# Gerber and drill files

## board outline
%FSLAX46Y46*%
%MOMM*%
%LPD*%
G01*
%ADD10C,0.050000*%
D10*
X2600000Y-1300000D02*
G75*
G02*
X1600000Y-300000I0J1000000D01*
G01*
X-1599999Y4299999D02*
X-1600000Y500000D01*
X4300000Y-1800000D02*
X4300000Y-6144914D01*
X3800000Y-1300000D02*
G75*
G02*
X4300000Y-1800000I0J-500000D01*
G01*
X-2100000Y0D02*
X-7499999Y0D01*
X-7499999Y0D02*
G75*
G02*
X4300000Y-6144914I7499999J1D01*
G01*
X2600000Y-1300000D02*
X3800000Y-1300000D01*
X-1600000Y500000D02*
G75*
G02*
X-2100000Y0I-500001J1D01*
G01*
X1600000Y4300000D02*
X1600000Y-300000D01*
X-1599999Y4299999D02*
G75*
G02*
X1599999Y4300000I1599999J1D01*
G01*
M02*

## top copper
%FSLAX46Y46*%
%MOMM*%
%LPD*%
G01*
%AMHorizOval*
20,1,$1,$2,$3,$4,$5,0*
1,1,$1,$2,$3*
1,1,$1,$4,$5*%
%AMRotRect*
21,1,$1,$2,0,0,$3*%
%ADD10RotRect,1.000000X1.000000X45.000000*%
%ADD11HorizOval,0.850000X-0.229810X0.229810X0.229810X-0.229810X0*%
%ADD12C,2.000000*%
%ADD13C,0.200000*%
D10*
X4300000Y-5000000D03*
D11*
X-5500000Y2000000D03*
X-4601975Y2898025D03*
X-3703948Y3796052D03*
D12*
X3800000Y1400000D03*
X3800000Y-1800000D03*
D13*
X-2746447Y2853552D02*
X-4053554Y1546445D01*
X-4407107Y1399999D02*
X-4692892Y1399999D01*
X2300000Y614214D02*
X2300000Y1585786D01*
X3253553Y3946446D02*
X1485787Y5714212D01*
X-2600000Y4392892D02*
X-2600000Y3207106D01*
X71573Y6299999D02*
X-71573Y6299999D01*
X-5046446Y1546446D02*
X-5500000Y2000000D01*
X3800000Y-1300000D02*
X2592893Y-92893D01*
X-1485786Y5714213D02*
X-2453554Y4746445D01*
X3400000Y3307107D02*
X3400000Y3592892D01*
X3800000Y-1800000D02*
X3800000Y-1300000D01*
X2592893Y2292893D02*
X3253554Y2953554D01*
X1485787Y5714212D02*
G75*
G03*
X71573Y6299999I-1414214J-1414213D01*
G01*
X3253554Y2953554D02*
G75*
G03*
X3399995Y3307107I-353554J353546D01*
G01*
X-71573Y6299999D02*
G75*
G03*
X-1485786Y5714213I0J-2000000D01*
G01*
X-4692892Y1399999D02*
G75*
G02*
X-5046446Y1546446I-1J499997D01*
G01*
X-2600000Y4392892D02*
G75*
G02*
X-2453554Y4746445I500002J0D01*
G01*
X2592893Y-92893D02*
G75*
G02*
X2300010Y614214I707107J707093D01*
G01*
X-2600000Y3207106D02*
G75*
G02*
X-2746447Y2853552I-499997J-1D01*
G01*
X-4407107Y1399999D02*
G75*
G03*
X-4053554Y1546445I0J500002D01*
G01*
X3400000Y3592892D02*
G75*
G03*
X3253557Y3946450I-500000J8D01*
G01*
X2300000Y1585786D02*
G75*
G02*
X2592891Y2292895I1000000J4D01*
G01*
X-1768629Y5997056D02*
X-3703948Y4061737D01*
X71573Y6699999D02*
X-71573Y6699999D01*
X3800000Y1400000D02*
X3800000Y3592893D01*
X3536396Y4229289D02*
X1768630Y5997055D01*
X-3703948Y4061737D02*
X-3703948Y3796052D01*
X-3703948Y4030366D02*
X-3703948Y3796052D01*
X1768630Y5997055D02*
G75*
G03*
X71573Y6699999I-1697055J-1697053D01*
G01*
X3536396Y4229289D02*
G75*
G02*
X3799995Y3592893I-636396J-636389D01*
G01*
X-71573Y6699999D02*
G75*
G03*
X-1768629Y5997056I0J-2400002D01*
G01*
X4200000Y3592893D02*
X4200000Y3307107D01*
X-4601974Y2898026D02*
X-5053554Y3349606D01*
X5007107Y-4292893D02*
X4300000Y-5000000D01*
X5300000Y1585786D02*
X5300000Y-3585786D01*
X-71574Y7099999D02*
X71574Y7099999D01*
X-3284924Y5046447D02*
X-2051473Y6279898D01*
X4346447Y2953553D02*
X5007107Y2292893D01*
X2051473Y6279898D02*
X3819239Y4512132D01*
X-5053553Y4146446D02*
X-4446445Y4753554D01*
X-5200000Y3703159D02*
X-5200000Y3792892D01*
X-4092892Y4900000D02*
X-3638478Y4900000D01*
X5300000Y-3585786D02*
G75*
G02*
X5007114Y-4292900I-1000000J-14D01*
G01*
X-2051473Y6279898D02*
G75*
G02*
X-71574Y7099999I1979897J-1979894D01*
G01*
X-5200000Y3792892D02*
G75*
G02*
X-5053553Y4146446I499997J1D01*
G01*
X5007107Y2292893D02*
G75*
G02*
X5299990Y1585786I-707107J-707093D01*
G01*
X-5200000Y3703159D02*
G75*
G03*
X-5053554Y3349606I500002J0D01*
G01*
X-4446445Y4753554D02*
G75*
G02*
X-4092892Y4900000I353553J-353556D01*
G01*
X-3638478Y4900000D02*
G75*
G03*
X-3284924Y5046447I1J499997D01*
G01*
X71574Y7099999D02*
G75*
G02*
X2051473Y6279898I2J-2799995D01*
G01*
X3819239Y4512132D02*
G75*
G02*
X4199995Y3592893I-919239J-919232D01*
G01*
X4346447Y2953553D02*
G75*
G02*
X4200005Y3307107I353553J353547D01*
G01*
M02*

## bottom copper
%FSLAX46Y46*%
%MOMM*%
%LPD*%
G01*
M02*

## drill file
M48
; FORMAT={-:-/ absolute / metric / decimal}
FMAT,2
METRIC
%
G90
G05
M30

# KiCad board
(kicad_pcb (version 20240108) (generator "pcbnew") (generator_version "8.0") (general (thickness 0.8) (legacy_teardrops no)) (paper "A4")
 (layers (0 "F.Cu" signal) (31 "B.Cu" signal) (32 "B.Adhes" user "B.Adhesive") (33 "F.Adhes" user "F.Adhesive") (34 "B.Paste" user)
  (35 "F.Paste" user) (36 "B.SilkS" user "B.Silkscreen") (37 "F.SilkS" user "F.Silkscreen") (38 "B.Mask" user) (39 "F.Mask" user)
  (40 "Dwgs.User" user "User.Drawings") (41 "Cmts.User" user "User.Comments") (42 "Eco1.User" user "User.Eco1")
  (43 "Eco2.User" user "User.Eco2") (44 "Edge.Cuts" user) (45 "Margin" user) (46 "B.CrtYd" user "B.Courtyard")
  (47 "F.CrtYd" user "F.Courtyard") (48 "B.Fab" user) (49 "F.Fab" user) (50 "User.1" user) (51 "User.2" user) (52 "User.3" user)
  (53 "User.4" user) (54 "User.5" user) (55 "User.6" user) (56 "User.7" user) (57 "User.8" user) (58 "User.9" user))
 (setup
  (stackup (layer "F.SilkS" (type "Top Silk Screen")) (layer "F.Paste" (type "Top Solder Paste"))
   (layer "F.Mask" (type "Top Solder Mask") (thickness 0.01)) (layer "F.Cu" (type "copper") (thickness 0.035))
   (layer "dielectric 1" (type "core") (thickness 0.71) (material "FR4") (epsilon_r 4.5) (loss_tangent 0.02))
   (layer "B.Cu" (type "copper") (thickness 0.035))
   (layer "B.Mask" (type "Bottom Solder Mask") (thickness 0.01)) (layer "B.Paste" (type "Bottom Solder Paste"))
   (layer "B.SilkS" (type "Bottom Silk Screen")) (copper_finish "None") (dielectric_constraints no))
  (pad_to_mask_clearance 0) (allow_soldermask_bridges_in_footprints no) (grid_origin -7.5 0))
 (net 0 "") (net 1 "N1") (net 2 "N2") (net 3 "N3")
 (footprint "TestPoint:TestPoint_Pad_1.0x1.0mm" (layer "F.Cu") (at 4.3 5 45)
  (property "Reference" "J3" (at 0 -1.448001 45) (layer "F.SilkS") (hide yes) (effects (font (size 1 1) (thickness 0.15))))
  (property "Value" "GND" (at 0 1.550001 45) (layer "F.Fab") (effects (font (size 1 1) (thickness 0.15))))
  (pad "1" smd rect (at 0 0 45) (size 1 1) (layers "F.Cu" "F.Mask") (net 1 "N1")))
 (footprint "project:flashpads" (layer "F.Cu") (at -4.601974 -2.898026 45)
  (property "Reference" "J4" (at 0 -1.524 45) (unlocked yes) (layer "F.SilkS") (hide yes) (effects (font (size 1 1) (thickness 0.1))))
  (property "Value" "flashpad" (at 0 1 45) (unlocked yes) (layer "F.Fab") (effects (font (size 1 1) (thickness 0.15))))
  (pad "1" smd oval (at -1.270001 0 135) (size 1.5 0.85) (layers "F.Cu" "F.Mask") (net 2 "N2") (thermal_bridge_angle 45))
  (pad "2" smd oval (at -0.000001 0 135) (size 1.5 0.85) (layers "F.Cu" "F.Mask") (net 1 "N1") (thermal_bridge_angle 45))
  (pad "3" smd oval (at 1.270001 0 135) (size 1.5 0.85) (layers "F.Cu" "F.Mask") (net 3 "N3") (thermal_bridge_angle 45)))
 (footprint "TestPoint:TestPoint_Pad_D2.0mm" (layer "F.Cu") (at 3.8 -1.4)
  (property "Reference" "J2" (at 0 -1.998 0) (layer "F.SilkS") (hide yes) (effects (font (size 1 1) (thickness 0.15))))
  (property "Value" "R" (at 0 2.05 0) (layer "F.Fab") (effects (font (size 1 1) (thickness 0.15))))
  (pad "1" smd circle (at 0 0) (size 2 2) (layers "F.Cu" "F.Mask") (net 3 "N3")))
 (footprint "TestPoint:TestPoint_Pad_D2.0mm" (layer "F.Cu") (at 3.8 1.8)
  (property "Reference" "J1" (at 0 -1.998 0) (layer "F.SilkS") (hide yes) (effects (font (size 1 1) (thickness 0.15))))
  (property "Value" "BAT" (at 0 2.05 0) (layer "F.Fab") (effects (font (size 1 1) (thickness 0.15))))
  (pad "1" smd circle (at 0 0) (size 2 2) (layers "F.Cu" "F.Mask") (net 2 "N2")))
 (gr_arc (start 2.6 1.3) (mid 1.892893 1.007107) (end 1.6 0.3) (stroke (width 0.05) (type default)) (layer "Edge.Cuts"))
 (gr_line (start -1.599999 -4.299999) (end -1.6 -0.5) (stroke (width 0.05) (type default)) (layer "Edge.Cuts"))
 (gr_line (start 4.3 1.8) (end 4.3 6.144914) (stroke (width 0.05) (type default)) (layer "Edge.Cuts"))
 (gr_arc (start 3.8 1.3) (mid 4.153553 1.446447) (end 4.3 1.8) (stroke (width 0.05) (type default)) (layer "Edge.Cuts"))
 (gr_line (start -2.1 0) (end -7.499999 0) (stroke (width 0.05) (type default)) (layer "Edge.Cuts"))
 (gr_arc (start -7.499999 0) (mid 3.588549 -6.585766) (end 4.3 6.144914) (stroke (width 0.05) (type default)) (layer "Edge.Cuts"))
 (gr_line (start 2.6 1.3) (end 3.8 1.3) (stroke (width 0.05) (type default)) (layer "Edge.Cuts"))
 (gr_arc (start -1.6 -0.5) (mid -1.746447 -0.146447) (end -2.1 0) (stroke (width 0.05) (type default)) (layer "Edge.Cuts"))
 (gr_line (start 1.6 -4.3) (end 1.6 0.3) (stroke (width 0.05) (type default)) (layer "Edge.Cuts"))
 (gr_arc (start -1.599999 -4.299999) (mid 0 -5.899999) (end 1.6 -4.3) (stroke (width 0.05) (type default)) (layer "Edge.Cuts"))
 (segment (start -2.746447 -2.853552) (end -4.053554 -1.546445) (width 0.2) (layer "F.Cu") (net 2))
 (segment (start -4.407107 -1.399999) (end -4.692892 -1.399999) (width 0.2) (layer "F.Cu") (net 2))
 (segment (start 2.3 -0.614214) (end 2.3 -1.585786) (width 0.2) (layer "F.Cu") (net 2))
 (segment (start 3.253553 -3.946446) (end 1.485787 -5.714212) (width 0.2) (layer "F.Cu") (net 2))
 (segment (start -2.6 -4.392892) (end -2.6 -3.207106) (width 0.2) (layer "F.Cu") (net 2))
 (segment (start 0.071573 -6.299999) (end -0.071573 -6.299999) (width 0.2) (layer "F.Cu") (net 2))
 (segment (start -5.046446 -1.546446) (end -5.5 -2) (width 0.2) (layer "F.Cu") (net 2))
 (segment (start 3.8 1.3) (end 2.592893 0.092893) (width 0.2) (layer "F.Cu") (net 2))
 (segment (start -1.485786 -5.714213) (end -2.453554 -4.746445) (width 0.2) (layer "F.Cu") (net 2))
 (segment (start 3.4 -3.307107) (end 3.4 -3.592892) (width 0.2) (layer "F.Cu") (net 2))
 (segment (start 3.8 1.8) (end 3.8 1.3) (width 0.2) (layer "F.Cu") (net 2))
 (segment (start 2.592893 -2.292893) (end 3.253554 -2.953554) (width 0.2) (layer "F.Cu") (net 2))
 (arc (start 1.485787 -5.714212) (mid 0.83694 -6.147758) (end 0.071573 -6.299999) (width 0.2) (layer "F.Cu") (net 2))
 (arc (start 3.253554 -2.953554) (mid 3.36194 -3.115766) (end 3.4 -3.307107) (width 0.2) (layer "F.Cu") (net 2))
 (arc (start -0.071573 -6.299999) (mid -0.83694 -6.147758) (end -1.485786 -5.714213) (width 0.2) (layer "F.Cu") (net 2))
 (arc (start -4.692892 -1.399999) (mid -4.884234 -1.438059) (end -5.046446 -1.546446) (width 0.2) (layer "F.Cu") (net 2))
 (arc (start -2.6 -4.392892) (mid -2.56194 -4.584233) (end -2.453554 -4.746445) (width 0.2) (layer "F.Cu") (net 2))
 (arc (start 2.592893 0.092893) (mid 2.37612 -0.231531) (end 2.3 -0.614214) (width 0.2) (layer "F.Cu") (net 2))
 (arc (start -2.6 -3.207106) (mid -2.63806 -3.015764) (end -2.746447 -2.853552) (width 0.2) (layer "F.Cu") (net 2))
 (arc (start -4.407107 -1.399999) (mid -4.215766 -1.438059) (end -4.053554 -1.546445) (width 0.2) (layer "F.Cu") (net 2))
 (arc (start 3.4 -3.592892) (mid 3.36194 -3.784234) (end 3.253553 -3.946446) (width 0.2) (layer "F.Cu") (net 2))
 (arc (start 2.3 -1.585786) (mid 2.37612 -1.968469) (end 2.592893 -2.292893) (width 0.2) (layer "F.Cu") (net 2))
 (segment (start -1.768629 -5.997056) (end -3.703948 -4.061737) (width 0.2) (layer "F.Cu") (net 3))
 (segment (start 0.071573 -6.699999) (end -0.071573 -6.699999) (width 0.2) (layer "F.Cu") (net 3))
 (segment (start 3.8 -1.4) (end 3.8 -3.592893) (width 0.2) (layer "F.Cu") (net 3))
 (segment (start 3.536396 -4.229289) (end 1.76863 -5.997055) (width 0.2) (layer "F.Cu") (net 3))
 (segment (start -3.703948 -4.061737) (end -3.703948 -3.796052) (width 0.2) (layer "F.Cu") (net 3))
 (segment (start -3.703948 -4.030366) (end -3.703948 -3.796052) (width 0.2) (layer "F.Cu") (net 3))
 (arc (start 1.76863 -5.997055) (mid 0.990014 -6.51731) (end 0.071573 -6.699999) (width 0.2) (layer "F.Cu") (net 3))
 (arc (start 3.536396 -4.229289) (mid 3.731491 -3.937308) (end 3.8 -3.592893) (width 0.2) (layer "F.Cu") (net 3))
 (arc (start -0.071573 -6.699999) (mid -0.990013 -6.51731) (end -1.768629 -5.997056) (width 0.2) (layer "F.Cu") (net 3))
 (segment (start 4.2 -3.592893) (end 4.2 -3.307107) (width 0.2) (layer "F.Cu") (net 1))
 (segment (start -4.601974 -2.898026) (end -5.053554 -3.349606) (width 0.2) (layer "F.Cu") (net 1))
 (segment (start 5.007107 4.292893) (end 4.3 5) (width 0.2) (layer "F.Cu") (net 1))
 (segment (start 5.3 -1.585786) (end 5.3 3.585786) (width 0.2) (layer "F.Cu") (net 1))
 (segment (start -0.071574 -7.099999) (end 0.071574 -7.099999) (width 0.2) (layer "F.Cu") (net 1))
 (segment (start -3.284924 -5.046447) (end -2.051473 -6.279898) (width 0.2) (layer "F.Cu") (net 1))
 (segment (start 4.346447 -2.953553) (end 5.007107 -2.292893) (width 0.2) (layer "F.Cu") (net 1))
 (segment (start 2.051473 -6.279898) (end 3.819239 -4.512132) (width 0.2) (layer "F.Cu") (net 1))
 (segment (start -5.053553 -4.146446) (end -4.446445 -4.753554) (width 0.2) (layer "F.Cu") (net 1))
 (segment (start -5.2 -3.703159) (end -5.2 -3.792892) (width 0.2) (layer "F.Cu") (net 1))
 (segment (start -4.092892 -4.9) (end -3.638478 -4.9) (width 0.2) (layer "F.Cu") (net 1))
 (arc (start 5.3 3.585786) (mid 5.22388 3.96847) (end 5.007107 4.292893) (width 0.2) (layer "F.Cu") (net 1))
 (arc (start -2.051473 -6.279898) (mid -1.143088 -6.886862) (end -0.071574 -7.099999) (width 0.2) (layer "F.Cu") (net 1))
 (arc (start -5.2 -3.792892) (mid -5.16194 -3.984234) (end -5.053553 -4.146446) (width 0.2) (layer "F.Cu") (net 1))
 (arc (start 5.007107 -2.292893) (mid 5.22388 -1.968469) (end 5.3 -1.585786) (width 0.2) (layer "F.Cu") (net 1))
 (arc (start -5.2 -3.703159) (mid -5.16194 -3.511818) (end -5.053554 -3.349606) (width 0.2) (layer "F.Cu") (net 1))
 (arc (start -4.446445 -4.753554) (mid -4.284233 -4.86194) (end -4.092892 -4.9) (width 0.2) (layer "F.Cu") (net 1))
 (arc (start -3.638478 -4.9) (mid -3.447136 -4.93806) (end -3.284924 -5.046447) (width 0.2) (layer "F.Cu") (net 1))
 (arc (start 0.071574 -7.099999) (mid 1.143088 -6.886862) (end 2.051473 -6.279898) (width 0.2) (layer "F.Cu") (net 1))
 (arc (start 3.819239 -4.512132) (mid 4.101044 -4.090382) (end 4.2 -3.592893) (width 0.2) (layer "F.Cu") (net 1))
 (arc (start 4.346447 -2.953553) (mid 4.23806 -3.115765) (end 4.2 -3.307107) (width 0.2) (layer "F.Cu") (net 1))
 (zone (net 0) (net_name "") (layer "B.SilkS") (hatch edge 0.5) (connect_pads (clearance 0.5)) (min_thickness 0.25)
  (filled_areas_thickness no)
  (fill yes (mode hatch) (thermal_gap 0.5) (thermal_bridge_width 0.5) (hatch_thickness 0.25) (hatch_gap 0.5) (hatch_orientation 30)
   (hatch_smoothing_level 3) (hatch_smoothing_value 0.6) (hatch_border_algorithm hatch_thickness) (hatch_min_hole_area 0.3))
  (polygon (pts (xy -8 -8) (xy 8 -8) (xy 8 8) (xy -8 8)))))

